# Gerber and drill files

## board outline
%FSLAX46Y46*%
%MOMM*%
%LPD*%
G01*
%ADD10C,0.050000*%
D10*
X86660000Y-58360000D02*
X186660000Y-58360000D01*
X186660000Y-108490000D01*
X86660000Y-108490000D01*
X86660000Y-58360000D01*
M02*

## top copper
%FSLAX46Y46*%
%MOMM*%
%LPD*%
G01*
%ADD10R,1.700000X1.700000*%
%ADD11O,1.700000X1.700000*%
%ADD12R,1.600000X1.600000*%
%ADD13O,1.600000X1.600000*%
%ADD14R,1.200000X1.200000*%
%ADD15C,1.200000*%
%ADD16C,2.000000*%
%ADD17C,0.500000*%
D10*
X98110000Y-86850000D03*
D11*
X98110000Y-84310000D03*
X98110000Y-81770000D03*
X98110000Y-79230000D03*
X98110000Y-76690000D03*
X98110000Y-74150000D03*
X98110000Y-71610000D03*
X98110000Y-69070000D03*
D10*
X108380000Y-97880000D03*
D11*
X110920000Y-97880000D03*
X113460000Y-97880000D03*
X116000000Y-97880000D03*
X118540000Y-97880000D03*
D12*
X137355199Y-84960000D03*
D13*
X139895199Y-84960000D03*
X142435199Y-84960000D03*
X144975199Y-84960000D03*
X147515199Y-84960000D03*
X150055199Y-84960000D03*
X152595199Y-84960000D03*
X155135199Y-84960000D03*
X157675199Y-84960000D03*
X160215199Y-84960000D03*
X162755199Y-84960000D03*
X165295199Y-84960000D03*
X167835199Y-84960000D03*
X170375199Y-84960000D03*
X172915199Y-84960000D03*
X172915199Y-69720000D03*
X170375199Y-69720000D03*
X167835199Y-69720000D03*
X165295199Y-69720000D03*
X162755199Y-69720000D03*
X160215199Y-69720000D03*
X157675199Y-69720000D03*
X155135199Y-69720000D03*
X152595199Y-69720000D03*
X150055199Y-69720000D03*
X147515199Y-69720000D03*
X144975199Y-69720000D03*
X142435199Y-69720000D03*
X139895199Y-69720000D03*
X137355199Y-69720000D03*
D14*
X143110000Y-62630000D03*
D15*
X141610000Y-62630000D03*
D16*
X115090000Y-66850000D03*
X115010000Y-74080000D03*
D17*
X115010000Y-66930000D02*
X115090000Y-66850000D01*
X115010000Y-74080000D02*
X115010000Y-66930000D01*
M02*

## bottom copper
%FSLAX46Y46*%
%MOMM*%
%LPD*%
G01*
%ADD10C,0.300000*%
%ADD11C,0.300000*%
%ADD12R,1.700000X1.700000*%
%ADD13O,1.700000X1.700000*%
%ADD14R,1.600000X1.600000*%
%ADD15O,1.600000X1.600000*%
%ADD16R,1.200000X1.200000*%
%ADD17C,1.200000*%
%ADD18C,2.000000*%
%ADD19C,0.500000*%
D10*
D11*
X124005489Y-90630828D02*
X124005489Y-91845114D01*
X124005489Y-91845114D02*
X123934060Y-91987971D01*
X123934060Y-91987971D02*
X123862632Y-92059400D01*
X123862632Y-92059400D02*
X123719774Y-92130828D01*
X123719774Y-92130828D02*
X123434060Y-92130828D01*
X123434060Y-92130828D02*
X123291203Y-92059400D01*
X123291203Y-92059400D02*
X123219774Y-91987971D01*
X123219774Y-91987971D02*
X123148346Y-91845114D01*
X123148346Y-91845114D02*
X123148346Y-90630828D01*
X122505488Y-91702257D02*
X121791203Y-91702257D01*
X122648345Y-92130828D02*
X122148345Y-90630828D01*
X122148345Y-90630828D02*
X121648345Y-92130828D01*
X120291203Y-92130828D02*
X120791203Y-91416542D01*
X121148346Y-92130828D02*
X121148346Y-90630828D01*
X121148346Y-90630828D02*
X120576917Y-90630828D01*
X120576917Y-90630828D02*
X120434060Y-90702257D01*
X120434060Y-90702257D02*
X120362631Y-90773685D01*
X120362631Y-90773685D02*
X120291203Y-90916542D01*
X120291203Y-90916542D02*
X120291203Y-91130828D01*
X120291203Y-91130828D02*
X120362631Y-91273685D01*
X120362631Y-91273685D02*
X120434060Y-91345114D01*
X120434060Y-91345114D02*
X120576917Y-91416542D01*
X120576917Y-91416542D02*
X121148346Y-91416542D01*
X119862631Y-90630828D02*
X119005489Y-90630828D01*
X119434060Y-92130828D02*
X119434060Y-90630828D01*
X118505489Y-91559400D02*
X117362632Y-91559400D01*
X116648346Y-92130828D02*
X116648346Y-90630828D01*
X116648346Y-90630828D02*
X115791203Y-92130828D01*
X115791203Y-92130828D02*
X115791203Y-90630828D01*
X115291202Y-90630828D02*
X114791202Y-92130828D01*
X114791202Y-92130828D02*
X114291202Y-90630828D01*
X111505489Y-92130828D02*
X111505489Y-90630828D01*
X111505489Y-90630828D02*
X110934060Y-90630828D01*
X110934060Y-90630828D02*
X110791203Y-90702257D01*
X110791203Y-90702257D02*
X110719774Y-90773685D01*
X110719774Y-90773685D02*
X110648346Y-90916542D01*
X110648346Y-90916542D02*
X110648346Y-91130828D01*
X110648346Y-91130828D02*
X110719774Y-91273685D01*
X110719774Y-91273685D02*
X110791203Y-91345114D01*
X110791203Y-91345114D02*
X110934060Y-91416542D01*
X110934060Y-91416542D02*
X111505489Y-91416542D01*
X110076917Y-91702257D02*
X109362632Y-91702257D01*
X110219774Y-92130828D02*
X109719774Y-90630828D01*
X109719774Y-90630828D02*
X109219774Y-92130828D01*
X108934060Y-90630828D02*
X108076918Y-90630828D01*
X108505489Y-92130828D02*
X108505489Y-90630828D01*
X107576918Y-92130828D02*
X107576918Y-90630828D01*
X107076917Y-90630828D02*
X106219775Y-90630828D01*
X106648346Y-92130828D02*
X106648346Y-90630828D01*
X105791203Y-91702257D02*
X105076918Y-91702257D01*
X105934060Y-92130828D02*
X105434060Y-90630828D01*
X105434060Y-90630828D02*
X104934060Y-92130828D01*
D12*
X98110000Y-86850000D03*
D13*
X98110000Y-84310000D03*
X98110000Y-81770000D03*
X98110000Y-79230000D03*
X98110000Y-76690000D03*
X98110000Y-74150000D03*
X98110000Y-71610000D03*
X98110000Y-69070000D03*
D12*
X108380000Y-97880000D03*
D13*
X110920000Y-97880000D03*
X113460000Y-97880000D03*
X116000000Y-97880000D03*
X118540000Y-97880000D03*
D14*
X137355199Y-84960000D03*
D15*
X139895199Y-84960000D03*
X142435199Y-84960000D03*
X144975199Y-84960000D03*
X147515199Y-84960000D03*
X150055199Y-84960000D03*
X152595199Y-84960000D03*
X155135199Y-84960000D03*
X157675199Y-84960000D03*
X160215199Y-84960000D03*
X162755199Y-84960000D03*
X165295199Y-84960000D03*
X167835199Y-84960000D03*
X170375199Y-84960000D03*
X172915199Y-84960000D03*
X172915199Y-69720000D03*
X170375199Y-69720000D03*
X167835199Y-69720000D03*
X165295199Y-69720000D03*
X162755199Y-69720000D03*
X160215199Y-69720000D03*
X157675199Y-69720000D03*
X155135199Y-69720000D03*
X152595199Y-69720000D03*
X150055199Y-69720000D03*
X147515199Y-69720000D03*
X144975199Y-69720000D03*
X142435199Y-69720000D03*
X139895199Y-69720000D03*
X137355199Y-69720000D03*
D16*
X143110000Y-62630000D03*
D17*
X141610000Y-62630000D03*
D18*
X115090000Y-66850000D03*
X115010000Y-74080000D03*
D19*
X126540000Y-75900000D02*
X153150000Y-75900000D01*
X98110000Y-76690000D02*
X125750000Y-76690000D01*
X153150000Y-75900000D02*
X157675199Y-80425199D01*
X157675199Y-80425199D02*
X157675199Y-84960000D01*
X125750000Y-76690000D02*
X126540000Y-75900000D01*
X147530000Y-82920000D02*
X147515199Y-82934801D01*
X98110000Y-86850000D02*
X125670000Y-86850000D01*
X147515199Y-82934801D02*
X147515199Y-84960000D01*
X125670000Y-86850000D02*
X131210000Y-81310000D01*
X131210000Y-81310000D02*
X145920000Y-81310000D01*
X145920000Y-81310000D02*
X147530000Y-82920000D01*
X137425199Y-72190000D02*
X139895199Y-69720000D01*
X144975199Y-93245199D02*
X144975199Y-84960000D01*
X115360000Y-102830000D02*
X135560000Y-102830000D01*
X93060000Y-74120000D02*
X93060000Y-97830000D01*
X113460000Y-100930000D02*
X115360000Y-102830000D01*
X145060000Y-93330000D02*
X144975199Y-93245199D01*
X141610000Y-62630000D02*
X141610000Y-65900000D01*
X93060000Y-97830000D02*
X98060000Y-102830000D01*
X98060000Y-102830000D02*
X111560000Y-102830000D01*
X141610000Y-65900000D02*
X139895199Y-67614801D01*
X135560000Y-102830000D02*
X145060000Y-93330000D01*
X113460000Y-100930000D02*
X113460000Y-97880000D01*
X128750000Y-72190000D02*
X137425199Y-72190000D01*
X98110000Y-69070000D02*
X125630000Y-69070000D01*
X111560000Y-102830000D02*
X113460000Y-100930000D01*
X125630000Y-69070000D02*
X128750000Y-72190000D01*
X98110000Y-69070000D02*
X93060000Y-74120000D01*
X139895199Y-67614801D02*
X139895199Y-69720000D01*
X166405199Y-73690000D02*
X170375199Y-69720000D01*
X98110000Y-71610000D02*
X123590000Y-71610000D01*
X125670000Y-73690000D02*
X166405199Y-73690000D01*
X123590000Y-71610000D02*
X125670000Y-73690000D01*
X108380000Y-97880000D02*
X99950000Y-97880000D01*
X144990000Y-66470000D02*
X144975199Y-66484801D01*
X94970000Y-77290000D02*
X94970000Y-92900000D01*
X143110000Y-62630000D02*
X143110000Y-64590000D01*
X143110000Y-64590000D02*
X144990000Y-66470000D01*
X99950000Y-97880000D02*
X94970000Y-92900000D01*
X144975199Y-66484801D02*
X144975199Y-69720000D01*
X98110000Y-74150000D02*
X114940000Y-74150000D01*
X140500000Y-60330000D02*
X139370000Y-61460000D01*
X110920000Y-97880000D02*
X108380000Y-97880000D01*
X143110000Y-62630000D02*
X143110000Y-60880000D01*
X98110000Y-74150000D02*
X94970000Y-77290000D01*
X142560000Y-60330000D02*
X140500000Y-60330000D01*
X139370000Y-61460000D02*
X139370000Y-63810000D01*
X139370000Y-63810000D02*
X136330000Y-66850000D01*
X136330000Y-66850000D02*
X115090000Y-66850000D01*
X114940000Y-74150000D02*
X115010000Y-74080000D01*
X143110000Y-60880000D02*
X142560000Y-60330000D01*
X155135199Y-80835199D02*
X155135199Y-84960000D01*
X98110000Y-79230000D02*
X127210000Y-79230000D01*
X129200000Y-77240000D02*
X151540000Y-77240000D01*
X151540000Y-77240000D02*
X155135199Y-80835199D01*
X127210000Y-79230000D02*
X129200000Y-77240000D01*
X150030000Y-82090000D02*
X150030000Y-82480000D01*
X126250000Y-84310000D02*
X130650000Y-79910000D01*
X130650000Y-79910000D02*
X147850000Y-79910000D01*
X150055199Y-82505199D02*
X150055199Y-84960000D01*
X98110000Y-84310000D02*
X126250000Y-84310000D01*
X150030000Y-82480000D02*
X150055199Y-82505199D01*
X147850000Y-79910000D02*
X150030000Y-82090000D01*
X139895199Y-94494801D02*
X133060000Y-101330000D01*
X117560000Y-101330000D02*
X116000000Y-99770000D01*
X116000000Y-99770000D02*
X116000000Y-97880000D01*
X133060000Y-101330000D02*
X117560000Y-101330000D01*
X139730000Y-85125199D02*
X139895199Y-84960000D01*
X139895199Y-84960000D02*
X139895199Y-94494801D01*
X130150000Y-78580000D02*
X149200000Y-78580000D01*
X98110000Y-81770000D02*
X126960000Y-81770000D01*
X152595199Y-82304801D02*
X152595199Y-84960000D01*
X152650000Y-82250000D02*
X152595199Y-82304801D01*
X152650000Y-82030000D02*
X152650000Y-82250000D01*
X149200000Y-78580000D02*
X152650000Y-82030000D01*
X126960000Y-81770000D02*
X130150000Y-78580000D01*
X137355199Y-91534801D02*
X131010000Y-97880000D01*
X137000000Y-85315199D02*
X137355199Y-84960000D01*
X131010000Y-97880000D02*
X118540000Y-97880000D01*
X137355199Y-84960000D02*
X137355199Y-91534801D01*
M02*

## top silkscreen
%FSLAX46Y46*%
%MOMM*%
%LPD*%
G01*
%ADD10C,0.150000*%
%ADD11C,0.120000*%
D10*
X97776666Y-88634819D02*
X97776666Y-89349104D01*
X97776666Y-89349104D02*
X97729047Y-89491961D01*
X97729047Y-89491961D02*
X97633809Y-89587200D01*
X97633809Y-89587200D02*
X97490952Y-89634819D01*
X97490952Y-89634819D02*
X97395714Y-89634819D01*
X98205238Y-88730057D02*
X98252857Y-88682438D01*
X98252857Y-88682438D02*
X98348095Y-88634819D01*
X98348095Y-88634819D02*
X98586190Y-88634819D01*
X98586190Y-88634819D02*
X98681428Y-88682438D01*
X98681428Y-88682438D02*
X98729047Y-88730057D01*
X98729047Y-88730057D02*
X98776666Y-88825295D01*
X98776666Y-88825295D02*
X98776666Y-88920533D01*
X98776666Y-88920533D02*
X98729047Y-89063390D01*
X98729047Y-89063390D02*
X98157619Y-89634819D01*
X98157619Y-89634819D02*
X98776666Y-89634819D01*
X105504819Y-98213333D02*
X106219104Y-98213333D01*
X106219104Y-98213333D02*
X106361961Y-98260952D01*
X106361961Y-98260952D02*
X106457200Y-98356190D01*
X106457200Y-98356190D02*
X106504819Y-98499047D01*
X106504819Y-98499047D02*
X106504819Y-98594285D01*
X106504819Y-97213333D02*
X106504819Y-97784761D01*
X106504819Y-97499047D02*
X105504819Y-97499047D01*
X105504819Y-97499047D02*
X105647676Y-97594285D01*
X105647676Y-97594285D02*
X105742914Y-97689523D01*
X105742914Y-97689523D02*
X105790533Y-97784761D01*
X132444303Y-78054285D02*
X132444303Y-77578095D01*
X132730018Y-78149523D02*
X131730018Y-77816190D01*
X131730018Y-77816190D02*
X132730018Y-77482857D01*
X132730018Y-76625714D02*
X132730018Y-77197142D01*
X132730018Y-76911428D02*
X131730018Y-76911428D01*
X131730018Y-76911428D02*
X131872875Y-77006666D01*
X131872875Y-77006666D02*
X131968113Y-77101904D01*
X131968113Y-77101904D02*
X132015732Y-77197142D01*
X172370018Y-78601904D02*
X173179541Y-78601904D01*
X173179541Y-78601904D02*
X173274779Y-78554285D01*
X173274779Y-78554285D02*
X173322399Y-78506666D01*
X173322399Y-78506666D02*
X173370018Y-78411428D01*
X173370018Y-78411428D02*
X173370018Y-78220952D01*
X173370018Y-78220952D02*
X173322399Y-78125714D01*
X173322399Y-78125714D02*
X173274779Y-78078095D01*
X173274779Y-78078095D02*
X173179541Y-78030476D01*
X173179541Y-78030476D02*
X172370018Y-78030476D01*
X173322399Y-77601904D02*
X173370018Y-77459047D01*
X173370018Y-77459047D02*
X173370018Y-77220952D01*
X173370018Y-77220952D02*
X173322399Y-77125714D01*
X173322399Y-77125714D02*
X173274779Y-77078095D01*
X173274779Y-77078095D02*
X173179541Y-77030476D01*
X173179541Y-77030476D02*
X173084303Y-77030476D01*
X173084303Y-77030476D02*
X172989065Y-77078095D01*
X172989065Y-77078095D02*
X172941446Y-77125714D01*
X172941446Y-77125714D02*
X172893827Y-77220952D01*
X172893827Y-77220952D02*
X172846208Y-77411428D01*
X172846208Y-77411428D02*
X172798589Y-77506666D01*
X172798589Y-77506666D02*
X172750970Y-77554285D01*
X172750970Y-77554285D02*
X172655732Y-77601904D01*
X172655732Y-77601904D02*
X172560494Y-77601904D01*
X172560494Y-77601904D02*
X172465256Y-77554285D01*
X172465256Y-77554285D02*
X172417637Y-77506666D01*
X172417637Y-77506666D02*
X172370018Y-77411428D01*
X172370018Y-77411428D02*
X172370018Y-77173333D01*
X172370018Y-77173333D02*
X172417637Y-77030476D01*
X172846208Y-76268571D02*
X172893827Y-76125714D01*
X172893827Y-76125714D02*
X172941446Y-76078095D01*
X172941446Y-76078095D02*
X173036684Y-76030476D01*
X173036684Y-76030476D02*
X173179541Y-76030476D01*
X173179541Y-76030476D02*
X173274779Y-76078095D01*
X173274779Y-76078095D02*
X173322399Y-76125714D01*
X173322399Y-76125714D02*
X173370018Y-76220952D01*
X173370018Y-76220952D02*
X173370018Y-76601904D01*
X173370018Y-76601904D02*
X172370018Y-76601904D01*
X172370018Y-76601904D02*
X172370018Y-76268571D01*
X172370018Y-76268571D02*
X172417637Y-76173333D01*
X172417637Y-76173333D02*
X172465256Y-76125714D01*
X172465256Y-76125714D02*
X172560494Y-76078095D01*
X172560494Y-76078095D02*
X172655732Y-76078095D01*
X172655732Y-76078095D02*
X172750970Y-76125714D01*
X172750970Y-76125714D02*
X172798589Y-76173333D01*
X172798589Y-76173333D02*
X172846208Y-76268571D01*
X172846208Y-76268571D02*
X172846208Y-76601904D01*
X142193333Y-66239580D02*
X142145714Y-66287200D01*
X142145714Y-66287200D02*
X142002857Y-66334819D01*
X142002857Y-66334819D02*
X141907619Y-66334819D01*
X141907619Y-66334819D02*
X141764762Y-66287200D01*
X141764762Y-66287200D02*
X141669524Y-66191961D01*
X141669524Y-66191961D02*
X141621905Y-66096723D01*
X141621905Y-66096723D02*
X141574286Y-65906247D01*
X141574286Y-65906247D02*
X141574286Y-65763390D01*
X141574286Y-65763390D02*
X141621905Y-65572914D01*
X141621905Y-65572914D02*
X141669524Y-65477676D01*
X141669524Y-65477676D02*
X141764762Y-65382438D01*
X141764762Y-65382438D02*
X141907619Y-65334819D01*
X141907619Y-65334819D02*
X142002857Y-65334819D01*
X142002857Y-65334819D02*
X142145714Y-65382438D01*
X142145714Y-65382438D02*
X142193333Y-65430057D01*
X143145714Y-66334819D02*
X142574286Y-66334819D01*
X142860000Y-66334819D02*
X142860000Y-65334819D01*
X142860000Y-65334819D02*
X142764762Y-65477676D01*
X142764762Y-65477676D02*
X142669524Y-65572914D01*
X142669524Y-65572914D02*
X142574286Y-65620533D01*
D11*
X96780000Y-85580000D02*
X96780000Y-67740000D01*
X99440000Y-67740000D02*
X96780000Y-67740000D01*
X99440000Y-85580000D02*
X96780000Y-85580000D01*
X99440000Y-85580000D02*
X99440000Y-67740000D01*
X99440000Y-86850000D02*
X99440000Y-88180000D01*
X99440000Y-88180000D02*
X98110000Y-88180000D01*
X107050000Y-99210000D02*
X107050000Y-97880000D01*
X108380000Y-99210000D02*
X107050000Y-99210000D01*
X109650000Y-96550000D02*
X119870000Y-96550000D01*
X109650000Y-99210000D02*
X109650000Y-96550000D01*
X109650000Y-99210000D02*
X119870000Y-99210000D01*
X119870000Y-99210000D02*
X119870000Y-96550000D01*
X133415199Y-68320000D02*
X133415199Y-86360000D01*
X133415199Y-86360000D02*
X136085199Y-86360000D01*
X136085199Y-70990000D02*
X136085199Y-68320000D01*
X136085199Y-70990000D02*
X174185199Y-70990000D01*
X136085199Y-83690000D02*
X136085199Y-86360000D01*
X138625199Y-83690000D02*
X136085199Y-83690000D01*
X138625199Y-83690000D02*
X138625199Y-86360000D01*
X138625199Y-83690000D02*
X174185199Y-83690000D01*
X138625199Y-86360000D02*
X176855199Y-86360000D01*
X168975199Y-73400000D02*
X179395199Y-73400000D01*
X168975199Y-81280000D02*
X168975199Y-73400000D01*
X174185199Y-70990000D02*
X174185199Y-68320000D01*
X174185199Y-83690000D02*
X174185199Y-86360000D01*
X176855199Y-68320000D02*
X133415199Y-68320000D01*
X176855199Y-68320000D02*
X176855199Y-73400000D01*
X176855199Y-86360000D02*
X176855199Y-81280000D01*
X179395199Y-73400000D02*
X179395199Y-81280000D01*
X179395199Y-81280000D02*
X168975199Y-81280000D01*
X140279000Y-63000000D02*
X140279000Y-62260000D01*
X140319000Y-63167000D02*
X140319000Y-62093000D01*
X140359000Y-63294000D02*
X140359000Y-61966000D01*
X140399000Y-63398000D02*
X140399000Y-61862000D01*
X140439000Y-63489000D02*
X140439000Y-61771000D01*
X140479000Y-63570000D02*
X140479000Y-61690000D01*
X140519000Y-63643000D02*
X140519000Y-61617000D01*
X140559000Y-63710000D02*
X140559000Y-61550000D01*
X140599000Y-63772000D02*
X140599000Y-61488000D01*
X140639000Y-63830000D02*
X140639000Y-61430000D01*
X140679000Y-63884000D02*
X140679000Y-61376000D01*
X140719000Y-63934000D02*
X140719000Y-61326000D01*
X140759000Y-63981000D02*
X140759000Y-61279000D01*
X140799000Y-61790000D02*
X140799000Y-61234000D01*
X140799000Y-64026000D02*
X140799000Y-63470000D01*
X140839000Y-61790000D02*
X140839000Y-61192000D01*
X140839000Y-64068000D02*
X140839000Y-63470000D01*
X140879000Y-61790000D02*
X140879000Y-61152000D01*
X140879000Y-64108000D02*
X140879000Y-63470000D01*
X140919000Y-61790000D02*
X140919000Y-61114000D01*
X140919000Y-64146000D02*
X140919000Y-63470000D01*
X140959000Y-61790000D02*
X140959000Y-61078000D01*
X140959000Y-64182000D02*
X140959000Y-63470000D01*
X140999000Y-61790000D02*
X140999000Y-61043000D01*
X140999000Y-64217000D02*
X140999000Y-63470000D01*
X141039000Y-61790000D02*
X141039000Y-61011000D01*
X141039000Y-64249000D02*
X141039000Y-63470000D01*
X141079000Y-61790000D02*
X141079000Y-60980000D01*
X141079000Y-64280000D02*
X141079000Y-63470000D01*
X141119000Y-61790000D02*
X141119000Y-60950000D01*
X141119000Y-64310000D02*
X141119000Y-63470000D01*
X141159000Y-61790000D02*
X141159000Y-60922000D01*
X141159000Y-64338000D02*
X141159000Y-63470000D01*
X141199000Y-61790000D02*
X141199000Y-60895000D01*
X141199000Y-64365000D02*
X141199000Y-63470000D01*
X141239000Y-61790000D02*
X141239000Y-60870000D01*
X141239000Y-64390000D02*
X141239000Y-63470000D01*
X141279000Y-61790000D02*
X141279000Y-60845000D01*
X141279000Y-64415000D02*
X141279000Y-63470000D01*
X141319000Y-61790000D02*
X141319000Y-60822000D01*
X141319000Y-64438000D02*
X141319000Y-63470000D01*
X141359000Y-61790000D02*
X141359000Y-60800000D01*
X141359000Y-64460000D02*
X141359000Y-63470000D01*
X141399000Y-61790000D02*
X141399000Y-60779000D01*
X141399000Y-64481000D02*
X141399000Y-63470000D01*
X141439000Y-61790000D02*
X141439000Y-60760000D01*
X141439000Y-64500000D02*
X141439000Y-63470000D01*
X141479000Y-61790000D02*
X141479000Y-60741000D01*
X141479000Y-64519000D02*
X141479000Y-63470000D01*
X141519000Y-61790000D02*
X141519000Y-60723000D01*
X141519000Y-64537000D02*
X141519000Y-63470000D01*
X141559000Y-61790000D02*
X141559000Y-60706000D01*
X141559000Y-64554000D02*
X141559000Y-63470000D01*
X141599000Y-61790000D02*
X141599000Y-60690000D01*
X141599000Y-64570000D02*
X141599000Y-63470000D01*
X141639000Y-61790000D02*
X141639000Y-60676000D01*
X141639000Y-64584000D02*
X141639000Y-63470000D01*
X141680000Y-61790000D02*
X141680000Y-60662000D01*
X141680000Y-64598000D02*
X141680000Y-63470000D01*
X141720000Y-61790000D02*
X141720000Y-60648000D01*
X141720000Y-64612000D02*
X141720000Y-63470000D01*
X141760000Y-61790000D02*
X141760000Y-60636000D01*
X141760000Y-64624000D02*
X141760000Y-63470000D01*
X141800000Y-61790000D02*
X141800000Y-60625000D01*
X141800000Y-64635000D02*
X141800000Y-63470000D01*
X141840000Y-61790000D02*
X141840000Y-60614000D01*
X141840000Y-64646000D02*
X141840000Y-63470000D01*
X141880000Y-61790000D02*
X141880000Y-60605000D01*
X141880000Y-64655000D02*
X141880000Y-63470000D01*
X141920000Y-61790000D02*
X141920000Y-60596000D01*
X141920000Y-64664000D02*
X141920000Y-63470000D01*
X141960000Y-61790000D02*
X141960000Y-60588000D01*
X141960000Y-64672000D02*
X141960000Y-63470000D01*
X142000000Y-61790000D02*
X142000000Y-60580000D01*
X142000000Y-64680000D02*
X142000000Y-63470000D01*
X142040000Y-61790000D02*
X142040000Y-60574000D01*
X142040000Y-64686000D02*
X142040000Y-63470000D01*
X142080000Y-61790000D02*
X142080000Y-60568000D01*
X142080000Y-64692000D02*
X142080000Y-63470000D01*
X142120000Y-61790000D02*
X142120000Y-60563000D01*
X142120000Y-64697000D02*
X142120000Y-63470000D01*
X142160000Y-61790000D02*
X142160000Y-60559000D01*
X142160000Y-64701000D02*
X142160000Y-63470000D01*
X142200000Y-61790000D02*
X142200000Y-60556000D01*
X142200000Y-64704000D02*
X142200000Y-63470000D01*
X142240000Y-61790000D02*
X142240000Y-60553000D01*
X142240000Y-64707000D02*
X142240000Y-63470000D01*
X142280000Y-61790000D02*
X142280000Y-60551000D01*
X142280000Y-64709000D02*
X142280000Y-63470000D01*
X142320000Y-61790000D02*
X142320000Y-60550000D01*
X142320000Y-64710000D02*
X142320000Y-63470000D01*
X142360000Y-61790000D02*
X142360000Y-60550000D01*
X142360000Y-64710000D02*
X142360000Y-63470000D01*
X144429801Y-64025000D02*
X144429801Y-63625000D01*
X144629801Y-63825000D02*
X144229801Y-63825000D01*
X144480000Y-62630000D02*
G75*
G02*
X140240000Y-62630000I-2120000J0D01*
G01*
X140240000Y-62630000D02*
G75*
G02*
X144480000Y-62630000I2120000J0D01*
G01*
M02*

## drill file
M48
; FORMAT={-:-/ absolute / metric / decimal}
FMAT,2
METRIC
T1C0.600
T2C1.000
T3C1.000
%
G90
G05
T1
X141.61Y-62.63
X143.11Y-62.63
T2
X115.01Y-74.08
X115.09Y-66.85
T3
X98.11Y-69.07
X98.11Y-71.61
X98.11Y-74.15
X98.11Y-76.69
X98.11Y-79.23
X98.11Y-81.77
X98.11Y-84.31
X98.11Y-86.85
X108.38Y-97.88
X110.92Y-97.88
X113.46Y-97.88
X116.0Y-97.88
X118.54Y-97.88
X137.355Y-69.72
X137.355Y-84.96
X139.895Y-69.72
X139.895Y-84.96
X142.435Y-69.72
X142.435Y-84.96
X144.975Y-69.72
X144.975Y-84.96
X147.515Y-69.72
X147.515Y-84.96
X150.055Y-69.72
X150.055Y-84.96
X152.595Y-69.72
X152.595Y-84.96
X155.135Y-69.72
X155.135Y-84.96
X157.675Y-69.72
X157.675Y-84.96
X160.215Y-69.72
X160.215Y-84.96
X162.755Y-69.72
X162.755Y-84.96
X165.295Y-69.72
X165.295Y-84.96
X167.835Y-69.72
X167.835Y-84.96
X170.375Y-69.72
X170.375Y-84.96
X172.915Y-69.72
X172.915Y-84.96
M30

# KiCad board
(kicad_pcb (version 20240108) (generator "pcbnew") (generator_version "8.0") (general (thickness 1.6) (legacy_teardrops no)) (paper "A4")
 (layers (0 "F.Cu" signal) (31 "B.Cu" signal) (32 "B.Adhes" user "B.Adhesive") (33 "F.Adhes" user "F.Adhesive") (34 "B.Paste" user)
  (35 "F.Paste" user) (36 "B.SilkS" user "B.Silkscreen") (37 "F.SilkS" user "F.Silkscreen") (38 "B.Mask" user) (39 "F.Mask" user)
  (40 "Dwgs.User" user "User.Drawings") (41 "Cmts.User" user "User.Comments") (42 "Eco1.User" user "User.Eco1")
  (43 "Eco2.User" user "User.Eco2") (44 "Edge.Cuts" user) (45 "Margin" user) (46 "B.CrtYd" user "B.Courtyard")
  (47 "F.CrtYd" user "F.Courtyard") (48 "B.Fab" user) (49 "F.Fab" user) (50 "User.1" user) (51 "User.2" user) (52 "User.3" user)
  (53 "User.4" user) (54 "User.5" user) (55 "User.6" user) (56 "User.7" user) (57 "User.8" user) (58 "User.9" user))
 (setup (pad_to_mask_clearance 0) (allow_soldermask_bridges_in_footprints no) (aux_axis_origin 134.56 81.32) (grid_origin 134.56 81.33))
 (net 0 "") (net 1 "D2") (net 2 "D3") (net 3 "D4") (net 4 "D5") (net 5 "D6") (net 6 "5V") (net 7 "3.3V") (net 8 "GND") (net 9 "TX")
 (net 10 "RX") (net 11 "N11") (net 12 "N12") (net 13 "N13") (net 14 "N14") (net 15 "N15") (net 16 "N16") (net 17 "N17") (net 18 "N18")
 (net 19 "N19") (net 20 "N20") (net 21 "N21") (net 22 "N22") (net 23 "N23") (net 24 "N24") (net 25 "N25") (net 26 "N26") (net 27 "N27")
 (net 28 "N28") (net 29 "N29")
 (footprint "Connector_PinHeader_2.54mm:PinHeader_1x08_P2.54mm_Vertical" (layer "F.Cu") (at 98.11 86.85 180)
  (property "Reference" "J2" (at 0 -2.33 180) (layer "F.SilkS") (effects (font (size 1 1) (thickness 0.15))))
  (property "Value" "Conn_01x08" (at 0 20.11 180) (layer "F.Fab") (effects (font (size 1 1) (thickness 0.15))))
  (fp_line (start 1.33 1.27) (end 1.33 19.11) (stroke (width 0.12) (type solid)) (layer "F.SilkS"))
  (fp_line (start -1.33 19.11) (end 1.33 19.11) (stroke (width 0.12) (type solid)) (layer "F.SilkS"))
  (fp_line (start -1.33 1.27) (end 1.33 1.27) (stroke (width 0.12) (type solid)) (layer "F.SilkS"))
  (fp_line (start -1.33 1.27) (end -1.33 19.11) (stroke (width 0.12) (type solid)) (layer "F.SilkS"))
  (fp_line (start -1.33 0) (end -1.33 -1.33) (stroke (width 0.12) (type solid)) (layer "F.SilkS"))
  (fp_line (start -1.33 -1.33) (end 0 -1.33) (stroke (width 0.12) (type solid)) (layer "F.SilkS"))
  (pad "1" thru_hole rect (at 0 0 180) (size 1.7 1.7) (drill 1) (layers "*.Cu" "*.Mask") (remove_unused_layers no) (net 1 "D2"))
  (pad "2" thru_hole oval (at 0 2.54 180) (size 1.7 1.7) (drill 1) (layers "*.Cu" "*.Mask") (remove_unused_layers no) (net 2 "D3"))
  (pad "3" thru_hole oval (at 0 5.08 180) (size 1.7 1.7) (drill 1) (layers "*.Cu" "*.Mask") (remove_unused_layers no) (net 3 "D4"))
  (pad "4" thru_hole oval (at 0 7.62 180) (size 1.7 1.7) (drill 1) (layers "*.Cu" "*.Mask") (remove_unused_layers no) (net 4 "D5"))
  (pad "5" thru_hole oval (at 0 10.16 180) (size 1.7 1.7) (drill 1) (layers "*.Cu" "*.Mask") (remove_unused_layers no) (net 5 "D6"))
  (pad "6" thru_hole oval (at 0 12.7 180) (size 1.7 1.7) (drill 1) (layers "*.Cu" "*.Mask") (remove_unused_layers no) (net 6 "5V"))
  (pad "7" thru_hole oval (at 0 15.24 180) (size 1.7 1.7) (drill 1) (layers "*.Cu" "*.Mask") (remove_unused_layers no) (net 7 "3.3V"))
  (pad "8" thru_hole oval (at 0 17.78 180) (size 1.7 1.7) (drill 1) (layers "*.Cu" "*.Mask") (remove_unused_layers no) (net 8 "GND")))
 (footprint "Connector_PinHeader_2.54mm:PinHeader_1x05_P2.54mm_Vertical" (layer "F.Cu") (at 108.38 97.88 90)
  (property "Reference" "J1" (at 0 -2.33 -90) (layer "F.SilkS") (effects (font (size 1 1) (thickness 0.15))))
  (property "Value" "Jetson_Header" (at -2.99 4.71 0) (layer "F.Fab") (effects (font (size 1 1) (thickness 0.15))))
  (fp_line (start -1.33 -1.33) (end 0 -1.33) (stroke (width 0.12) (type solid)) (layer "F.SilkS"))
  (fp_line (start -1.33 0) (end -1.33 -1.33) (stroke (width 0.12) (type solid)) (layer "F.SilkS"))
  (fp_line (start 1.33 1.27) (end 1.33 11.49) (stroke (width 0.12) (type solid)) (layer "F.SilkS"))
  (fp_line (start -1.33 1.27) (end 1.33 1.27) (stroke (width 0.12) (type solid)) (layer "F.SilkS"))
  (fp_line (start -1.33 1.27) (end -1.33 11.49) (stroke (width 0.12) (type solid)) (layer "F.SilkS"))
  (fp_line (start -1.33 11.49) (end 1.33 11.49) (stroke (width 0.12) (type solid)) (layer "F.SilkS"))
  (pad "1" thru_hole rect (at 0 0 90) (size 1.7 1.7) (drill 1) (layers "*.Cu" "*.Mask") (remove_unused_layers no) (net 6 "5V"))
  (pad "2" thru_hole oval (at 0 2.54 90) (size 1.7 1.7) (drill 1) (layers "*.Cu" "*.Mask") (remove_unused_layers no) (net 6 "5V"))
  (pad "3" thru_hole oval (at 0 5.08 90) (size 1.7 1.7) (drill 1) (layers "*.Cu" "*.Mask") (remove_unused_layers no) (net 8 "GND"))
  (pad "4" thru_hole oval (at 0 7.62 90) (size 1.7 1.7) (drill 1) (layers "*.Cu" "*.Mask") (remove_unused_layers no) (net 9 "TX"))
  (pad "5" thru_hole oval (at 0 10.16 90) (size 1.7 1.7) (drill 1) (layers "*.Cu" "*.Mask") (remove_unused_layers no) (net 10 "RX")))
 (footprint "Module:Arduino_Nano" (layer "F.Cu") (at 137.355199 84.96 90)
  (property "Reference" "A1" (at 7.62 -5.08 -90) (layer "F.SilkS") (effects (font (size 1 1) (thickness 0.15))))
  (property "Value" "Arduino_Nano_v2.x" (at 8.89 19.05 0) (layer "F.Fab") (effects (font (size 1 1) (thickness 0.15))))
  (fp_line (start 16.64 -3.94) (end -1.4 -3.94) (stroke (width 0.12) (type solid)) (layer "F.SilkS"))
  (fp_line (start -1.4 -3.94) (end -1.4 -1.27) (stroke (width 0.12) (type solid)) (layer "F.SilkS"))
  (fp_line (start 13.97 -1.27) (end 16.64 -1.27) (stroke (width 0.12) (type solid)) (layer "F.SilkS"))
  (fp_line (start 13.97 -1.27) (end 13.97 36.83) (stroke (width 0.12) (type solid)) (layer "F.SilkS"))
  (fp_line (start 1.27 -1.27) (end -1.4 -1.27) (stroke (width 0.12) (type solid)) (layer "F.SilkS"))
  (fp_line (start 1.27 1.27) (end 1.27 -1.27) (stroke (width 0.12) (type solid)) (layer "F.SilkS"))
  (fp_line (start 1.27 1.27) (end -1.4 1.27) (stroke (width 0.12) (type solid)) (layer "F.SilkS"))
  (fp_line (start 1.27 1.27) (end 1.27 36.83) (stroke (width 0.12) (type solid)) (layer "F.SilkS"))
  (fp_line (start -1.4 1.27) (end -1.4 39.5) (stroke (width 0.12) (type solid)) (layer "F.SilkS"))
  (fp_line (start 11.56 31.62) (end 11.56 42.04) (stroke (width 0.12) (type solid)) (layer "F.SilkS"))
  (fp_line (start 3.68 31.62) (end 11.56 31.62) (stroke (width 0.12) (type solid)) (layer "F.SilkS"))
  (fp_line (start 13.97 36.83) (end 16.64 36.83) (stroke (width 0.12) (type solid)) (layer "F.SilkS"))
  (fp_line (start 1.27 36.83) (end -1.4 36.83) (stroke (width 0.12) (type solid)) (layer "F.SilkS"))
  (fp_line (start 16.64 39.5) (end 16.64 -3.94) (stroke (width 0.12) (type solid)) (layer "F.SilkS"))
  (fp_line (start 16.64 39.5) (end 11.56 39.5) (stroke (width 0.12) (type solid)) (layer "F.SilkS"))
  (fp_line (start -1.4 39.5) (end 3.68 39.5) (stroke (width 0.12) (type solid)) (layer "F.SilkS"))
  (fp_line (start 11.56 42.04) (end 3.68 42.04) (stroke (width 0.12) (type solid)) (layer "F.SilkS"))
  (fp_line (start 3.68 42.04) (end 3.68 31.62) (stroke (width 0.12) (type solid)) (layer "F.SilkS"))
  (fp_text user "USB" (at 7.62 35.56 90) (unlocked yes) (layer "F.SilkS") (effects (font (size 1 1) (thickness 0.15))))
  (pad "1" thru_hole rect (at 0 0 90) (size 1.6 1.6) (drill 1) (layers "*.Cu" "*.Mask") (remove_unused_layers no) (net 10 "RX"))
  (pad "2" thru_hole oval (at 0 2.54 90) (size 1.6 1.6) (drill 1) (layers "*.Cu" "*.Mask") (remove_unused_layers no) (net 9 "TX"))
  (pad "3" thru_hole oval (at 0 5.08 90) (size 1.6 1.6) (drill 1) (layers "*.Cu" "*.Mask") (remove_unused_layers no) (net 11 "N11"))
  (pad "4" thru_hole oval (at 0 7.62 90) (size 1.6 1.6) (drill 1) (layers "*.Cu" "*.Mask") (remove_unused_layers no) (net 8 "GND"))
  (pad "5" thru_hole oval (at 0 10.16 90) (size 1.6 1.6) (drill 1) (layers "*.Cu" "*.Mask") (remove_unused_layers no) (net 1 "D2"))
  (pad "6" thru_hole oval (at 0 12.7 90) (size 1.6 1.6) (drill 1) (layers "*.Cu" "*.Mask") (remove_unused_layers no) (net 2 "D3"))
  (pad "7" thru_hole oval (at 0 15.24 90) (size 1.6 1.6) (drill 1) (layers "*.Cu" "*.Mask") (remove_unused_layers no) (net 3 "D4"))
  (pad "8" thru_hole oval (at 0 17.78 90) (size 1.6 1.6) (drill 1) (layers "*.Cu" "*.Mask") (remove_unused_layers no) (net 4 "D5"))
  (pad "9" thru_hole oval (at 0 20.32 90) (size 1.6 1.6) (drill 1) (layers "*.Cu" "*.Mask") (remove_unused_layers no) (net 5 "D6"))
  (pad "10" thru_hole oval (at 0 22.86 90) (size 1.6 1.6) (drill 1) (layers "*.Cu" "*.Mask") (remove_unused_layers no) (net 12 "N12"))
  (pad "11" thru_hole oval (at 0 25.4 90) (size 1.6 1.6) (drill 1) (layers "*.Cu" "*.Mask") (remove_unused_layers no) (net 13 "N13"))
  (pad "12" thru_hole oval (at 0 27.94 90) (size 1.6 1.6) (drill 1) (layers "*.Cu" "*.Mask") (remove_unused_layers no) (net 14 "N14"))
  (pad "13" thru_hole oval (at 0 30.48 90) (size 1.6 1.6) (drill 1) (layers "*.Cu" "*.Mask") (remove_unused_layers no) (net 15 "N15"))
  (pad "14" thru_hole oval (at 0 33.02 90) (size 1.6 1.6) (drill 1) (layers "*.Cu" "*.Mask") (remove_unused_layers no) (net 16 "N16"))
  (pad "15" thru_hole oval (at 0 35.56 90) (size 1.6 1.6) (drill 1) (layers "*.Cu" "*.Mask") (remove_unused_layers no) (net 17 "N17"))
  (pad "16" thru_hole oval (at 15.24 35.56 90) (size 1.6 1.6) (drill 1) (layers "*.Cu" "*.Mask") (remove_unused_layers no) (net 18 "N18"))
  (pad "17" thru_hole oval (at 15.24 33.02 90) (size 1.6 1.6) (drill 1) (layers "*.Cu" "*.Mask") (remove_unused_layers no) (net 7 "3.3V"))
  (pad "18" thru_hole oval (at 15.24 30.48 90) (size 1.6 1.6) (drill 1) (layers "*.Cu" "*.Mask") (remove_unused_layers no) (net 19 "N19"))
  (pad "19" thru_hole oval (at 15.24 27.94 90) (size 1.6 1.6) (drill 1) (layers "*.Cu" "*.Mask") (remove_unused_layers no) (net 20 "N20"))
  (pad "20" thru_hole oval (at 15.24 25.4 90) (size 1.6 1.6) (drill 1) (layers "*.Cu" "*.Mask") (remove_unused_layers no) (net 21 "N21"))
  (pad "21" thru_hole oval (at 15.24 22.86 90) (size 1.6 1.6) (drill 1) (layers "*.Cu" "*.Mask") (remove_unused_layers no) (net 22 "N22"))
  (pad "22" thru_hole oval (at 15.24 20.32 90) (size 1.6 1.6) (drill 1) (layers "*.Cu" "*.Mask") (remove_unused_layers no) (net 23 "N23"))
  (pad "23" thru_hole oval (at 15.24 17.78 90) (size 1.6 1.6) (drill 1) (layers "*.Cu" "*.Mask") (remove_unused_layers no) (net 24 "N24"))
  (pad "24" thru_hole oval (at 15.24 15.24 90) (size 1.6 1.6) (drill 1) (layers "*.Cu" "*.Mask") (remove_unused_layers no) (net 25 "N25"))
  (pad "25" thru_hole oval (at 15.24 12.7 90) (size 1.6 1.6) (drill 1) (layers "*.Cu" "*.Mask") (remove_unused_layers no) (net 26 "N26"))
  (pad "26" thru_hole oval (at 15.24 10.16 90) (size 1.6 1.6) (drill 1) (layers "*.Cu" "*.Mask") (remove_unused_layers no) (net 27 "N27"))
  (pad "27" thru_hole oval (at 15.24 7.62 90) (size 1.6 1.6) (drill 1) (layers "*.Cu" "*.Mask") (remove_unused_layers no) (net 6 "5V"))
  (pad "28" thru_hole oval (at 15.24 5.08 90) (size 1.6 1.6) (drill 1) (layers "*.Cu" "*.Mask") (remove_unused_layers no) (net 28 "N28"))
  (pad "29" thru_hole oval (at 15.24 2.54 90) (size 1.6 1.6) (drill 1) (layers "*.Cu" "*.Mask") (remove_unused_layers no) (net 8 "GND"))
  (pad "30" thru_hole oval (at 15.24 0 90) (size 1.6 1.6) (drill 1) (layers "*.Cu" "*.Mask") (remove_unused_layers no) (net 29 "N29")))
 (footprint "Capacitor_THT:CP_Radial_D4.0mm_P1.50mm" (layer "F.Cu") (at 143.11 62.63 180)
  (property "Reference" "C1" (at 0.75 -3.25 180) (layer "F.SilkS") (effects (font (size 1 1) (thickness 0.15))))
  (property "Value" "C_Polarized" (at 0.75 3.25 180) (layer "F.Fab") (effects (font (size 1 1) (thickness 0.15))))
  (fp_line (start 2.831 -0.37) (end 2.831 0.37) (stroke (width 0.12) (type solid)) (layer "F.SilkS"))
  (fp_line (start 2.791 -0.537) (end 2.791 0.537) (stroke (width 0.12) (type solid)) (layer "F.SilkS"))
  (fp_line (start 2.751 -0.664) (end 2.751 0.664) (stroke (width 0.12) (type solid)) (layer "F.SilkS"))
  (fp_line (start 2.711 -0.768) (end 2.711 0.768) (stroke (width 0.12) (type solid)) (layer "F.SilkS"))
  (fp_line (start 2.671 -0.859) (end 2.671 0.859) (stroke (width 0.12) (type solid)) (layer "F.SilkS"))
  (fp_line (start 2.631 -0.94) (end 2.631 0.94) (stroke (width 0.12) (type solid)) (layer "F.SilkS"))
  (fp_line (start 2.591 -1.013) (end 2.591 1.013) (stroke (width 0.12) (type solid)) (layer "F.SilkS"))
  (fp_line (start 2.551 -1.08) (end 2.551 1.08) (stroke (width 0.12) (type solid)) (layer "F.SilkS"))
  (fp_line (start 2.511 -1.142) (end 2.511 1.142) (stroke (width 0.12) (type solid)) (layer "F.SilkS"))
  (fp_line (start 2.471 -1.2) (end 2.471 1.2) (stroke (width 0.12) (type solid)) (layer "F.SilkS"))
  (fp_line (start 2.431 -1.254) (end 2.431 1.254) (stroke (width 0.12) (type solid)) (layer "F.SilkS"))
  (fp_line (start 2.391 -1.304) (end 2.391 1.304) (stroke (width 0.12) (type solid)) (layer "F.SilkS"))
  (fp_line (start 2.351 -1.351) (end 2.351 1.351) (stroke (width 0.12) (type solid)) (layer "F.SilkS"))
  (fp_line (start 2.311 0.84) (end 2.311 1.396) (stroke (width 0.12) (type solid)) (layer "F.SilkS"))
  (fp_line (start 2.311 -1.396) (end 2.311 -0.84) (stroke (width 0.12) (type solid)) (layer "F.SilkS"))
  (fp_line (start 2.271 0.84) (end 2.271 1.438) (stroke (width 0.12) (type solid)) (layer "F.SilkS"))
  (fp_line (start 2.271 -1.438) (end 2.271 -0.84) (stroke (width 0.12) (type solid)) (layer "F.SilkS"))
  (fp_line (start 2.231 0.84) (end 2.231 1.478) (stroke (width 0.12) (type solid)) (layer "F.SilkS"))
  (fp_line (start 2.231 -1.478) (end 2.231 -0.84) (stroke (width 0.12) (type solid)) (layer "F.SilkS"))
  (fp_line (start 2.191 0.84) (end 2.191 1.516) (stroke (width 0.12) (type solid)) (layer "F.SilkS"))
  (fp_line (start 2.191 -1.516) (end 2.191 -0.84) (stroke (width 0.12) (type solid)) (layer "F.SilkS"))
  (fp_line (start 2.151 0.84) (end 2.151 1.552) (stroke (width 0.12) (type solid)) (layer "F.SilkS"))
  (fp_line (start 2.151 -1.552) (end 2.151 -0.84) (stroke (width 0.12) (type solid)) (layer "F.SilkS"))
  (fp_line (start 2.111 0.84) (end 2.111 1.587) (stroke (width 0.12) (type solid)) (layer "F.SilkS"))
  (fp_line (start 2.111 -1.587) (end 2.111 -0.84) (stroke (width 0.12) (type solid)) (layer "F.SilkS"))
  (fp_line (start 2.071 0.84) (end 2.071 1.619) (stroke (width 0.12) (type solid)) (layer "F.SilkS"))
  (fp_line (start 2.071 -1.619) (end 2.071 -0.84) (stroke (width 0.12) (type solid)) (layer "F.SilkS"))
  (fp_line (start 2.031 0.84) (end 2.031 1.65) (stroke (width 0.12) (type solid)) (layer "F.SilkS"))
  (fp_line (start 2.031 -1.65) (end 2.031 -0.84) (stroke (width 0.12) (type solid)) (layer "F.SilkS"))
  (fp_line (start 1.991 0.84) (end 1.991 1.68) (stroke (width 0.12) (type solid)) (layer "F.SilkS"))
  (fp_line (start 1.991 -1.68) (end 1.991 -0.84) (stroke (width 0.12) (type solid)) (layer "F.SilkS"))
  (fp_line (start 1.951 0.84) (end 1.951 1.708) (stroke (width 0.12) (type solid)) (layer "F.SilkS"))
  (fp_line (start 1.951 -1.708) (end 1.951 -0.84) (stroke (width 0.12) (type solid)) (layer "F.SilkS"))
  (fp_line (start 1.911 0.84) (end 1.911 1.735) (stroke (width 0.12) (type solid)) (layer "F.SilkS"))
  (fp_line (start 1.911 -1.735) (end 1.911 -0.84) (stroke (width 0.12) (type solid)) (layer "F.SilkS"))
  (fp_line (start 1.871 0.84) (end 1.871 1.76) (stroke (width 0.12) (type solid)) (layer "F.SilkS"))
  (fp_line (start 1.871 -1.76) (end 1.871 -0.84) (stroke (width 0.12) (type solid)) (layer "F.SilkS"))
  (fp_line (start 1.831 0.84) (end 1.831 1.785) (stroke (width 0.12) (type solid)) (layer "F.SilkS"))
  (fp_line (start 1.831 -1.785) (end 1.831 -0.84) (stroke (width 0.12) (type solid)) (layer "F.SilkS"))
  (fp_line (start 1.791 0.84) (end 1.791 1.808) (stroke (width 0.12) (type solid)) (layer "F.SilkS"))
  (fp_line (start 1.791 -1.808) (end 1.791 -0.84) (stroke (width 0.12) (type solid)) (layer "F.SilkS"))
  (fp_line (start 1.751 0.84) (end 1.751 1.83) (stroke (width 0.12) (type solid)) (layer "F.SilkS"))
  (fp_line (start 1.751 -1.83) (end 1.751 -0.84) (stroke (width 0.12) (type solid)) (layer "F.SilkS"))
  (fp_line (start 1.711 0.84) (end 1.711 1.851) (stroke (width 0.12) (type solid)) (layer "F.SilkS"))
  (fp_line (start 1.711 -1.851) (end 1.711 -0.84) (stroke (width 0.12) (type solid)) (layer "F.SilkS"))
  (fp_line (start 1.671 0.84) (end 1.671 1.87) (stroke (width 0.12) (type solid)) (layer "F.SilkS"))
  (fp_line (start 1.671 -1.87) (end 1.671 -0.84) (stroke (width 0.12) (type solid)) (layer "F.SilkS"))
  (fp_line (start 1.631 0.84) (end 1.631 1.889) (stroke (width 0.12) (type solid)) (layer "F.SilkS"))
  (fp_line (start 1.631 -1.889) (end 1.631 -0.84) (stroke (width 0.12) (type solid)) (layer "F.SilkS"))
  (fp_line (start 1.591 0.84) (end 1.591 1.907) (stroke (width 0.12) (type solid)) (layer "F.SilkS"))
  (fp_line (start 1.591 -1.907) (end 1.591 -0.84) (stroke (width 0.12) (type solid)) (layer "F.SilkS"))
  (fp_line (start 1.551 0.84) (end 1.551 1.924) (stroke (width 0.12) (type solid)) (layer "F.SilkS"))
  (fp_line (start 1.551 -1.924) (end 1.551 -0.84) (stroke (width 0.12) (type solid)) (layer "F.SilkS"))
  (fp_line (start 1.511 0.84) (end 1.511 1.94) (stroke (width 0.12) (type solid)) (layer "F.SilkS"))
  (fp_line (start 1.511 -1.94) (end 1.511 -0.84) (stroke (width 0.12) (type solid)) (layer "F.SilkS"))
  (fp_line (start 1.471 0.84) (end 1.471 1.954) (stroke (width 0.12) (type solid)) (layer "F.SilkS"))
  (fp_line (start 1.471 -1.954) (end 1.471 -0.84) (stroke (width 0.12) (type solid)) (layer "F.SilkS"))
  (fp_line (start 1.43 0.84) (end 1.43 1.968) (stroke (width 0.12) (type solid)) (layer "F.SilkS"))
  (fp_line (start 1.43 -1.968) (end 1.43 -0.84) (stroke (width 0.12) (type solid)) (layer "F.SilkS"))
  (fp_line (start 1.39 0.84) (end 1.39 1.982) (stroke (width 0.12) (type solid)) (layer "F.SilkS"))
  (fp_line (start 1.39 -1.982) (end 1.39 -0.84) (stroke (width 0.12) (type solid)) (layer "F.SilkS"))
  (fp_line (start 1.35 0.84) (end 1.35 1.994) (stroke (width 0.12) (type solid)) (layer "F.SilkS"))
  (fp_line (start 1.35 -1.994) (end 1.35 -0.84) (stroke (width 0.12) (type solid)) (layer "F.SilkS"))
  (fp_line (start 1.31 0.84) (end 1.31 2.005) (stroke (width 0.12) (type solid)) (layer "F.SilkS"))
  (fp_line (start 1.31 -2.005) (end 1.31 -0.84) (stroke (width 0.12) (type solid)) (layer "F.SilkS"))
  (fp_line (start 1.27 0.84) (end 1.27 2.016) (stroke (width 0.12) (type solid)) (layer "F.SilkS"))
  (fp_line (start 1.27 -2.016) (end 1.27 -0.84) (stroke (width 0.12) (type solid)) (layer "F.SilkS"))
  (fp_line (start 1.23 0.84) (end 1.23 2.025) (stroke (width 0.12) (type solid)) (layer "F.SilkS"))
  (fp_line (start 1.23 -2.025) (end 1.23 -0.84) (stroke (width 0.12) (type solid)) (layer "F.SilkS"))
  (fp_line (start 1.19 0.84) (end 1.19 2.034) (stroke (width 0.12) (type solid)) (layer "F.SilkS"))
  (fp_line (start 1.19 -2.034) (end 1.19 -0.84) (stroke (width 0.12) (type solid)) (layer "F.SilkS"))
  (fp_line (start 1.15 0.84) (end 1.15 2.042) (stroke (width 0.12) (type solid)) (layer "F.SilkS"))
  (fp_line (start 1.15 -2.042) (end 1.15 -0.84) (stroke (width 0.12) (type solid)) (layer "F.SilkS"))
  (fp_line (start 1.11 0.84) (end 1.11 2.05) (stroke (width 0.12) (type solid)) (layer "F.SilkS"))
  (fp_line (start 1.11 -2.05) (end 1.11 -0.84) (stroke (width 0.12) (type solid)) (layer "F.SilkS"))
  (fp_line (start 1.07 0.84) (end 1.07 2.056) (stroke (width 0.12) (type solid)) (layer "F.SilkS"))
  (fp_line (start 1.07 -2.056) (end 1.07 -0.84) (stroke (width 0.12) (type solid)) (layer "F.SilkS"))
  (fp_line (start 1.03 0.84) (end 1.03 2.062) (stroke (width 0.12) (type solid)) (layer "F.SilkS"))
  (fp_line (start 1.03 -2.062) (end 1.03 -0.84) (stroke (width 0.12) (type solid)) (layer "F.SilkS"))
  (fp_line (start 0.99 0.84) (end 0.99 2.067) (stroke (width 0.12) (type solid)) (layer "F.SilkS"))
  (fp_line (start 0.99 -2.067) (end 0.99 -0.84) (stroke (width 0.12) (type solid)) (layer "F.SilkS"))
  (fp_line (start 0.95 0.84) (end 0.95 2.071) (stroke (width 0.12) (type solid)) (layer "F.SilkS"))
  (fp_line (start 0.95 -2.071) (end 0.95 -0.84) (stroke (width 0.12) (type solid)) (layer "F.SilkS"))
  (fp_line (start 0.91 0.84) (end 0.91 2.074) (stroke (width 0.12) (type solid)) (layer "F.SilkS"))
  (fp_line (start 0.91 -2.074) (end 0.91 -0.84) (stroke (width 0.12) (type solid)) (layer "F.SilkS"))
  (fp_line (start 0.87 0.84) (end 0.87 2.077) (stroke (width 0.12) (type solid)) (layer "F.SilkS"))
  (fp_line (start 0.87 -2.077) (end 0.87 -0.84) (stroke (width 0.12) (type solid)) (layer "F.SilkS"))
  (fp_line (start 0.83 0.84) (end 0.83 2.079) (stroke (width 0.12) (type solid)) (layer "F.SilkS"))
  (fp_line (start 0.83 -2.079) (end 0.83 -0.84) (stroke (width 0.12) (type solid)) (layer "F.SilkS"))
  (fp_line (start 0.79 0.84) (end 0.79 2.08) (stroke (width 0.12) (type solid)) (layer "F.SilkS"))
  (fp_line (start 0.79 -2.08) (end 0.79 -0.84) (stroke (width 0.12) (type solid)) (layer "F.SilkS"))
  (fp_line (start 0.75 0.84) (end 0.75 2.08) (stroke (width 0.12) (type solid)) (layer "F.SilkS"))
  (fp_line (start 0.75 -2.08) (end 0.75 -0.84) (stroke (width 0.12) (type solid)) (layer "F.SilkS"))
  (fp_line (start -1.319801 -1.395) (end -1.319801 -0.995) (stroke (width 0.12) (type solid)) (layer "F.SilkS"))
  (fp_line (start -1.519801 -1.195) (end -1.119801 -1.195) (stroke (width 0.12) (type solid)) (layer "F.SilkS"))
  (fp_circle (center 0.75 0) (end 2.87 0) (stroke (width 0.12) (type solid)) (fill none) (layer "F.SilkS"))
  (pad "1" thru_hole rect (at 0 0 180) (size 1.2 1.2) (drill 0.6) (layers "*.Cu" "*.Mask") (remove_unused_layers no) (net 6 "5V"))
  (pad "2" thru_hole circle (at 1.5 0 180) (size 1.2 1.2) (drill 0.6) (layers "*.Cu" "*.Mask") (remove_unused_layers no) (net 8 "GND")))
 (gr_rect (start 86.66 58.36) (end 186.66 108.49) (stroke (width 0.05) (type default)) (fill none) (layer "Edge.Cuts"))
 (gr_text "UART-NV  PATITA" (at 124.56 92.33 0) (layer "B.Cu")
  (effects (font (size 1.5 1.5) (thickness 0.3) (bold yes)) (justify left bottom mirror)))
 (segment (start 126.54 75.9) (end 153.15 75.9) (width 0.5) (layer "B.Cu") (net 5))
 (segment (start 98.11 76.69) (end 125.75 76.69) (width 0.5) (layer "B.Cu") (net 5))
 (segment (start 153.15 75.9) (end 157.675199 80.425199) (width 0.5) (layer "B.Cu") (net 5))
 (segment (start 157.675199 80.425199) (end 157.675199 84.96) (width 0.5) (layer "B.Cu") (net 5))
 (segment (start 125.75 76.69) (end 126.54 75.9) (width 0.5) (layer "B.Cu") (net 5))
 (segment (start 147.53 82.92) (end 147.515199 82.934801) (width 0.5) (layer "B.Cu") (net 1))
 (segment (start 98.11 86.85) (end 125.67 86.85) (width 0.5) (layer "B.Cu") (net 1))
 (segment (start 147.515199 82.934801) (end 147.515199 84.96) (width 0.5) (layer "B.Cu") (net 1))
 (segment (start 125.67 86.85) (end 131.21 81.31) (width 0.5) (layer "B.Cu") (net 1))
 (segment (start 131.21 81.31) (end 145.92 81.31) (width 0.5) (layer "B.Cu") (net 1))
 (segment (start 145.92 81.31) (end 147.53 82.92) (width 0.5) (layer "B.Cu") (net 1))
 (segment (start 137.425199 72.19) (end 139.895199 69.72) (width 0.5) (layer "B.Cu") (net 8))
 (segment (start 144.975199 93.245199) (end 144.975199 84.96) (width 0.5) (layer "B.Cu") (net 8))
 (segment (start 115.36 102.83) (end 135.56 102.83) (width 0.5) (layer "B.Cu") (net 8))
 (segment (start 93.06 74.12) (end 93.06 97.83) (width 0.5) (layer "B.Cu") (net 8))
 (segment (start 113.46 100.93) (end 115.36 102.83) (width 0.5) (layer "B.Cu") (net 8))
 (segment (start 145.06 93.33) (end 144.975199 93.245199) (width 0.5) (layer "B.Cu") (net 8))
 (segment (start 141.61 62.63) (end 141.61 65.9) (width 0.5) (layer "B.Cu") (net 8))
 (segment (start 93.06 97.83) (end 98.06 102.83) (width 0.5) (layer "B.Cu") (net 8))
 (segment (start 98.06 102.83) (end 111.56 102.83) (width 0.5) (layer "B.Cu") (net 8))
 (segment (start 141.61 65.9) (end 139.895199 67.614801) (width 0.5) (layer "B.Cu") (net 8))
 (segment (start 135.56 102.83) (end 145.06 93.33) (width 0.5) (layer "B.Cu") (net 8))
 (segment (start 113.46 100.93) (end 113.46 97.88) (width 0.5) (layer "B.Cu") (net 8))
 (segment (start 128.75 72.19) (end 137.425199 72.19) (width 0.5) (layer "B.Cu") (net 8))
 (segment (start 98.11 69.07) (end 125.63 69.07) (width 0.5) (layer "B.Cu") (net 8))
 (segment (start 111.56 102.83) (end 113.46 100.93) (width 0.5) (layer "B.Cu") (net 8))
 (segment (start 125.63 69.07) (end 128.75 72.19) (width 0.5) (layer "B.Cu") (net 8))
 (segment (start 98.11 69.07) (end 93.06 74.12) (width 0.5) (layer "B.Cu") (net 8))
 (segment (start 139.895199 67.614801) (end 139.895199 69.72) (width 0.5) (layer "B.Cu") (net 8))
 (segment (start 166.405199 73.69) (end 170.375199 69.72) (width 0.5) (layer "B.Cu") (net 7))
 (segment (start 98.11 71.61) (end 123.59 71.61) (width 0.5) (layer "B.Cu") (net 7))
 (segment (start 125.67 73.69) (end 166.405199 73.69) (width 0.5) (layer "B.Cu") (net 7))
 (segment (start 123.59 71.61) (end 125.67 73.69) (width 0.5) (layer "B.Cu") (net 7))
 (segment (start 115.01 66.93) (end 115.09 66.85) (width 0.5) (layer "F.Cu") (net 6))
 (segment (start 115.01 74.08) (end 115.01 66.93) (width 0.5) (layer "F.Cu") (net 6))
 (via (at 115.09 66.85) (size 2) (drill 1) (layers "F.Cu" "B.Cu") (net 6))
 (via (at 115.01 74.08) (size 2) (drill 1) (layers "F.Cu" "B.Cu") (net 6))
 (segment (start 108.38 97.88) (end 99.95 97.88) (width 0.5) (layer "B.Cu") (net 6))
 (segment (start 144.99 66.47) (end 144.975199 66.484801) (width 0.5) (layer "B.Cu") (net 6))
 (segment (start 94.97 77.29) (end 94.97 92.9) (width 0.5) (layer "B.Cu") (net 6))
 (segment (start 143.11 62.63) (end 143.11 64.59) (width 0.5) (layer "B.Cu") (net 6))
 (segment (start 143.11 64.59) (end 144.99 66.47) (width 0.5) (layer "B.Cu") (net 6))
 (segment (start 99.95 97.88) (end 94.97 92.9) (width 0.5) (layer "B.Cu") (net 6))
 (segment (start 144.975199 66.484801) (end 144.975199 69.72) (width 0.5) (layer "B.Cu") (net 6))
 (segment (start 98.11 74.15) (end 114.94 74.15) (width 0.5) (layer "B.Cu") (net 6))
 (segment (start 140.5 60.33) (end 139.37 61.46) (width 0.5) (layer "B.Cu") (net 6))
 (segment (start 110.92 97.88) (end 108.38 97.88) (width 0.5) (layer "B.Cu") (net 6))
 (segment (start 143.11 62.63) (end 143.11 60.88) (width 0.5) (layer "B.Cu") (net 6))
 (segment (start 98.11 74.15) (end 94.97 77.29) (width 0.5) (layer "B.Cu") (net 6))
 (segment (start 142.56 60.33) (end 140.5 60.33) (width 0.5) (layer "B.Cu") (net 6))
 (segment (start 139.37 61.46) (end 139.37 63.81) (width 0.5) (layer "B.Cu") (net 6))
 (segment (start 139.37 63.81) (end 136.33 66.85) (width 0.5) (layer "B.Cu") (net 6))
 (segment (start 136.33 66.85) (end 115.09 66.85) (width 0.5) (layer "B.Cu") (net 6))
 (segment (start 114.94 74.15) (end 115.01 74.08) (width 0.5) (layer "B.Cu") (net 6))
 (segment (start 143.11 60.88) (end 142.56 60.33) (width 0.5) (layer "B.Cu") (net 6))
 (segment (start 155.135199 80.835199) (end 155.135199 84.96) (width 0.5) (layer "B.Cu") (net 4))
 (segment (start 98.11 79.23) (end 127.21 79.23) (width 0.5) (layer "B.Cu") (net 4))
 (segment (start 129.2 77.24) (end 151.54 77.24) (width 0.5) (layer "B.Cu") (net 4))
 (segment (start 151.54 77.24) (end 155.135199 80.835199) (width 0.5) (layer "B.Cu") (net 4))
 (segment (start 127.21 79.23) (end 129.2 77.24) (width 0.5) (layer "B.Cu") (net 4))
 (segment (start 150.03 82.09) (end 150.03 82.48) (width 0.5) (layer "B.Cu") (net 2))
 (segment (start 126.25 84.31) (end 130.65 79.91) (width 0.5) (layer "B.Cu") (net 2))
 (segment (start 130.65 79.91) (end 147.85 79.91) (width 0.5) (layer "B.Cu") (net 2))
 (segment (start 150.055199 82.505199) (end 150.055199 84.96) (width 0.5) (layer "B.Cu") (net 2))
 (segment (start 98.11 84.31) (end 126.25 84.31) (width 0.5) (layer "B.Cu") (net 2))
 (segment (start 150.03 82.48) (end 150.055199 82.505199) (width 0.5) (layer "B.Cu") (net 2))
 (segment (start 147.85 79.91) (end 150.03 82.09) (width 0.5) (layer "B.Cu") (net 2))
 (segment (start 139.895199 94.494801) (end 133.06 101.33) (width 0.5) (layer "B.Cu") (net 9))
 (segment (start 117.56 101.33) (end 116 99.77) (width 0.5) (layer "B.Cu") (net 9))
 (segment (start 116 99.77) (end 116 97.88) (width 0.5) (layer "B.Cu") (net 9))
 (segment (start 133.06 101.33) (end 117.56 101.33) (width 0.5) (layer "B.Cu") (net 9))
 (segment (start 139.73 85.125199) (end 139.895199 84.96) (width 0.5) (layer "B.Cu") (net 9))
 (segment (start 139.895199 84.96) (end 139.895199 94.494801) (width 0.5) (layer "B.Cu") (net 9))
 (segment (start 130.15 78.58) (end 149.2 78.58) (width 0.5) (layer "B.Cu") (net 3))
 (segment (start 98.11 81.77) (end 126.96 81.77) (width 0.5) (layer "B.Cu") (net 3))
 (segment (start 152.595199 82.304801) (end 152.595199 84.96) (width 0.5) (layer "B.Cu") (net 3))
 (segment (start 152.65 82.25) (end 152.595199 82.304801) (width 0.5) (layer "B.Cu") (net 3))
 (segment (start 152.65 82.03) (end 152.65 82.25) (width 0.5) (layer "B.Cu") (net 3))
 (segment (start 149.2 78.58) (end 152.65 82.03) (width 0.5) (layer "B.Cu") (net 3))
 (segment (start 126.96 81.77) (end 130.15 78.58) (width 0.5) (layer "B.Cu") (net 3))
 (segment (start 137.355199 91.534801) (end 131.01 97.88) (width 0.5) (layer "B.Cu") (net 10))
 (segment (start 137 85.315199) (end 137.355199 84.96) (width 0.5) (layer "B.Cu") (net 10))
 (segment (start 131.01 97.88) (end 118.54 97.88) (width 0.5) (layer "B.Cu") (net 10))
 (segment (start 137.355199 84.96) (end 137.355199 91.534801) (width 0.5) (layer "B.Cu") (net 10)))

